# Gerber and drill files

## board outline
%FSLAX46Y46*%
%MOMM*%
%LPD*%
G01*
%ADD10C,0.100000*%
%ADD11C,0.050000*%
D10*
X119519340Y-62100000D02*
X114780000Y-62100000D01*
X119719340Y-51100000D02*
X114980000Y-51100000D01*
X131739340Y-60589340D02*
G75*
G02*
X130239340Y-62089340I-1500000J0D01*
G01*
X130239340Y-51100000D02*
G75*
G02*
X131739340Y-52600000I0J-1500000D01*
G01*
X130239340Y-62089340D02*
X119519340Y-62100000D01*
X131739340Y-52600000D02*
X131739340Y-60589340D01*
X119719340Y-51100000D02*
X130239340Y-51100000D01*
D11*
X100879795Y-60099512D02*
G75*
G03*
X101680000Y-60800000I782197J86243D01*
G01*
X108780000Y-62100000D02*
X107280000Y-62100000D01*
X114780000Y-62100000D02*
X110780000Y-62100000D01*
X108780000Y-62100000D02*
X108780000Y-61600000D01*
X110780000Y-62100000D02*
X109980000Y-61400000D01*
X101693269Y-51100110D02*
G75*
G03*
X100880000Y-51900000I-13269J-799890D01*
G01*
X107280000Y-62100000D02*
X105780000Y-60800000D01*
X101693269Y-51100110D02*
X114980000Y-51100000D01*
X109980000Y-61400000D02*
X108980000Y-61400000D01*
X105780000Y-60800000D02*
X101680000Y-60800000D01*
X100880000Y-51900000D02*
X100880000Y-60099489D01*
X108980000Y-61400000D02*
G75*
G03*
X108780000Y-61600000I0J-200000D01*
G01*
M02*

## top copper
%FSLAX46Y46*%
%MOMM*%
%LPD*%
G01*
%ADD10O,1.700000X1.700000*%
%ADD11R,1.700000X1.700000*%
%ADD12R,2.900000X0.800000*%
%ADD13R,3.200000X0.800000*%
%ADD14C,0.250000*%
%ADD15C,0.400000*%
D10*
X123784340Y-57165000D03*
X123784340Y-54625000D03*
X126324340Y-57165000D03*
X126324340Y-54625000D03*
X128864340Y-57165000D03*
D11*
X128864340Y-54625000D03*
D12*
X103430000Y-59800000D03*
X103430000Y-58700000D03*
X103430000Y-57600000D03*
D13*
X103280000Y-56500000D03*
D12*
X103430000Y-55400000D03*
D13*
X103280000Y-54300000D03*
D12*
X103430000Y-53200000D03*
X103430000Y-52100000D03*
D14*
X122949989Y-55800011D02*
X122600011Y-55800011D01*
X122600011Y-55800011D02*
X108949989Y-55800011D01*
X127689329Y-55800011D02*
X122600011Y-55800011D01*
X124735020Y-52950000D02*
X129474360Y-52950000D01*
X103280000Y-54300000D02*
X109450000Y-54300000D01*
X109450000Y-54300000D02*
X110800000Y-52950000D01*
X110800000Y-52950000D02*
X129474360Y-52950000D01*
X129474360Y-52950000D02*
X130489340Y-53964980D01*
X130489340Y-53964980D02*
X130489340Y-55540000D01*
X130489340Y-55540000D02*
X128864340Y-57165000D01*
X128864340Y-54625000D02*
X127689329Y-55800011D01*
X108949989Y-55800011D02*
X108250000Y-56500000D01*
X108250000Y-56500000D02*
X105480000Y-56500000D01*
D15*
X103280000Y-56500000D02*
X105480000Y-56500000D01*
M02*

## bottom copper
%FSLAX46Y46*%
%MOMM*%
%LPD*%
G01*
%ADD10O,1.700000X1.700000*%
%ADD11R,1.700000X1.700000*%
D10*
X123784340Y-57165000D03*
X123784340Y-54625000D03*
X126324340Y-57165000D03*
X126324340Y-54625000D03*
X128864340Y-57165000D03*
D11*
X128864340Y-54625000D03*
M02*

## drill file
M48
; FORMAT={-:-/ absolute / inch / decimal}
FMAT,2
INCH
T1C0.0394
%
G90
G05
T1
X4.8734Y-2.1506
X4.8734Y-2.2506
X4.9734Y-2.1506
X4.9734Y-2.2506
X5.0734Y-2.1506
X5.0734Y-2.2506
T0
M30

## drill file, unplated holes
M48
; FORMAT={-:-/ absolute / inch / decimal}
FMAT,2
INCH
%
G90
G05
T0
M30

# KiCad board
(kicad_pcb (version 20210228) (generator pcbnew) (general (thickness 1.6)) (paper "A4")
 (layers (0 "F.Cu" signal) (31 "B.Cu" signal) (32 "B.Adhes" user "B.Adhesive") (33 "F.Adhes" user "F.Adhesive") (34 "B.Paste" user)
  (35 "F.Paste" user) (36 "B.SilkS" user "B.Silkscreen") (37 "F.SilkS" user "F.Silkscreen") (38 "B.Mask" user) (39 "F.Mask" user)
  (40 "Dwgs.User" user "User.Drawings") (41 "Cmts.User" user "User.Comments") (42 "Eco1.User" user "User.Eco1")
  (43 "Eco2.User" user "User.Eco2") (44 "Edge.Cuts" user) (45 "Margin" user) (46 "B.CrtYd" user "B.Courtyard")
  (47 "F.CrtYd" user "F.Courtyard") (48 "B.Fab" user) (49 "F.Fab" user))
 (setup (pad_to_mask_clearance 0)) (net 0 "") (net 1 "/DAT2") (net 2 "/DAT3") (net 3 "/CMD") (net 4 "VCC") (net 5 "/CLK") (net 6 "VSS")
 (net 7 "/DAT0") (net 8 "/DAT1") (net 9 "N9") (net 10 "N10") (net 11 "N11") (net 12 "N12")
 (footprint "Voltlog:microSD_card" (layer "F.Cu") (at 109.63 55.95 90)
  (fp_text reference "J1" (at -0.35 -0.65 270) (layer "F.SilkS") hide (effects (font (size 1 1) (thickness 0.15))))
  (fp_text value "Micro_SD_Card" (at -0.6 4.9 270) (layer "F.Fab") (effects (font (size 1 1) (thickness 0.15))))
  (pad "1" smd rect (at -3.85 -6.2 90) (locked) (size 0.8 2.9) (layers "F.Cu" "F.Mask") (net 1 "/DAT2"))
  (pad "2" smd rect (at -2.75 -6.2 90) (locked) (size 0.8 2.9) (layers "F.Cu" "F.Mask") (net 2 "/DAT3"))
  (pad "3" smd rect (at -1.65 -6.2 90) (locked) (size 0.8 2.9) (layers "F.Cu" "F.Mask") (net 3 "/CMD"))
  (pad "4" smd rect (at -0.55 -6.35 90) (locked) (size 0.8 3.2) (layers "F.Cu" "F.Mask") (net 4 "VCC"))
  (pad "5" smd rect (at 0.55 -6.2 90) (locked) (size 0.8 2.9) (layers "F.Cu" "F.Mask") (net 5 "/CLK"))
  (pad "6" smd rect (at 1.65 -6.35 90) (locked) (size 0.8 3.2) (layers "F.Cu" "F.Mask") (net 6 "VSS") (zone_connect 2))
  (pad "7" smd rect (at 2.75 -6.2 90) (locked) (size 0.8 2.9) (layers "F.Cu" "F.Mask") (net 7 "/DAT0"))
  (pad "8" smd rect (at 3.85 -6.2 90) (locked) (size 0.8 2.9) (layers "F.Cu" "F.Mask") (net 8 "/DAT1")))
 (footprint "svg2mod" (layer "F.Cu") (at 115.55 56.15)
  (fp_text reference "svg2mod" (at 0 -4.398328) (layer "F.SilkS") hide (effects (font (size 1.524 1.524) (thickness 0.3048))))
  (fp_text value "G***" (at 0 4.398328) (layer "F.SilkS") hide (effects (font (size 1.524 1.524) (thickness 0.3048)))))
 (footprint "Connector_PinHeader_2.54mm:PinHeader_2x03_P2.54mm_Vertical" (layer "F.Cu") (at 128.86434 54.625 -90)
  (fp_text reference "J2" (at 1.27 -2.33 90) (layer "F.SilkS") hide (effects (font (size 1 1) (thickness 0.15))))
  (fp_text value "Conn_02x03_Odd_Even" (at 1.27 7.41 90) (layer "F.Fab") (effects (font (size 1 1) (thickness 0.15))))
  (pad "1" thru_hole rect (at 0 0 270) (locked) (size 1.7 1.7) (drill 1) (layers *.Cu *.Mask) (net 4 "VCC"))
  (pad "2" thru_hole oval (at 2.54 0 270) (locked) (size 1.7 1.7) (drill 1) (layers *.Cu *.Mask) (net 6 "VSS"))
  (pad "3" thru_hole oval (at 0 2.54 270) (locked) (size 1.7 1.7) (drill 1) (layers *.Cu *.Mask) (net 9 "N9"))
  (pad "4" thru_hole oval (at 2.54 2.54 270) (locked) (size 1.7 1.7) (drill 1) (layers *.Cu *.Mask) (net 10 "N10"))
  (pad "5" thru_hole oval (at 0 5.08 270) (locked) (size 1.7 1.7) (drill 1) (layers *.Cu *.Mask) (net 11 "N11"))
  (pad "6" thru_hole oval (at 2.54 5.08 270) (locked) (size 1.7 1.7) (drill 1) (layers *.Cu *.Mask) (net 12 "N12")))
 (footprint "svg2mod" (layer "F.Cu") (at 121.35 60.4)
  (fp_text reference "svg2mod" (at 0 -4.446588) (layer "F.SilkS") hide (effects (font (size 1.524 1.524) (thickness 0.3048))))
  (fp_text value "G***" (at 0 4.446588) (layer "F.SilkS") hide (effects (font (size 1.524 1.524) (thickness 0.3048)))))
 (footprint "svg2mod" (layer "F.Cu") (at 115.55 53.35)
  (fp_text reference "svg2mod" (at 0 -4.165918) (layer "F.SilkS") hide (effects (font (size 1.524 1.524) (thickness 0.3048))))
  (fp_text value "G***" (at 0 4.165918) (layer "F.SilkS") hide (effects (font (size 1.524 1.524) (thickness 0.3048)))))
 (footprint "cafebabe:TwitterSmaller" (layer "B.Cu") (at 120.4 60 180)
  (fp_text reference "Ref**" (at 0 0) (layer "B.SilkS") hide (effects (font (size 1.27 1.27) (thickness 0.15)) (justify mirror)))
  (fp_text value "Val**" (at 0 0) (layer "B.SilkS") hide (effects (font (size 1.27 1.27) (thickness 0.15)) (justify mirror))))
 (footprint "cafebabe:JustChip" (layer "B.Cu") (at 113 55.9 180)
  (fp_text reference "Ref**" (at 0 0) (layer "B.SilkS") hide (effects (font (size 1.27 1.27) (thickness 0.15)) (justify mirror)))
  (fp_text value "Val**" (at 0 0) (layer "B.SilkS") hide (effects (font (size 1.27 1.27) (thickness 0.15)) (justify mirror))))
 (gr_arc (start 101.661992 60.013269) (end 101.68 60.8) (angle 85.01938241) (layer "Edge.Cuts") (width 0.05))
 (gr_line (start 108.78 62.1) (end 107.28 62.1) (layer "Edge.Cuts") (width 0.05))
 (gr_line (start 119.71934 51.1) (end 114.98 51.1) (layer "Edge.Cuts") (width 0.1))
 (gr_line (start 119.71934 51.1) (end 130.23934 51.1) (layer "Edge.Cuts") (width 0.1))
 (gr_line (start 119.51934 62.1) (end 114.78 62.1) (layer "Edge.Cuts") (width 0.1))
 (gr_line (start 114.78 62.1) (end 110.78 62.1) (layer "Edge.Cuts") (width 0.05))
 (gr_arc (start 130.23934 60.58934) (end 130.23934 62.08934) (angle -90) (layer "Edge.Cuts") (width 0.1))
 (gr_line (start 108.78 62.1) (end 108.78 61.6) (layer "Edge.Cuts") (width 0.05))
 (gr_line (start 110.78 62.1) (end 109.98 61.4) (layer "Edge.Cuts") (width 0.05))
 (gr_arc (start 101.68 51.9) (end 100.88 51.9) (angle 90.95033288) (layer "Edge.Cuts") (width 0.05))
 (gr_line (start 107.28 62.1) (end 105.78 60.8) (layer "Edge.Cuts") (width 0.05))
 (gr_line (start 101.693269 51.10011) (end 114.98 51.1) (layer "Edge.Cuts") (width 0.05))
 (gr_line (start 109.98 61.4) (end 108.98 61.4) (layer "Edge.Cuts") (width 0.05))
 (gr_line (start 105.78 60.8) (end 101.68 60.8) (layer "Edge.Cuts") (width 0.05))
 (gr_line (start 131.73934 52.6) (end 131.73934 60.58934) (layer "Edge.Cuts") (width 0.1))
 (gr_arc (start 130.23934 52.6) (end 131.73934 52.6) (angle -90) (layer "Edge.Cuts") (width 0.1))
 (gr_line (start 100.88 51.9) (end 100.88 60.099489) (layer "Edge.Cuts") (width 0.05))
 (gr_arc (start 108.98 61.6) (end 108.78 61.6) (angle 90) (layer "Edge.Cuts") (width 0.05))
 (gr_line (start 130.23934 62.08934) (end 119.51934 62.1) (layer "Edge.Cuts") (width 0.1))
 (segment (start 122.949989 55.800011) (end 122.600011 55.800011) (width 0.25) (layer "F.Cu") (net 4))
 (segment (start 128.86434 54.625) (end 127.689329 55.800011) (width 0.25) (layer "F.Cu") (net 4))
 (segment (start 127.689329 55.800011) (end 122.600011 55.800011) (width 0.25) (layer "F.Cu") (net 4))
 (segment (start 122.600011 55.800011) (end 108.949989 55.800011) (width 0.25) (layer "F.Cu") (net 4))
 (segment (start 108.25 56.5) (end 105.48 56.5) (width 0.25) (layer "F.Cu") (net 4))
 (segment (start 108.949989 55.800011) (end 108.25 56.5) (width 0.25) (layer "F.Cu") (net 4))
 (segment (start 103.28 56.5) (end 105.48 56.5) (width 0.4) (layer "F.Cu") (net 4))
 (segment (start 109.45 54.3) (end 110.8 52.95) (width 0.25) (layer "F.Cu") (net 6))
 (segment (start 103.28 54.3) (end 109.45 54.3) (width 0.25) (layer "F.Cu") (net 6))
 (segment (start 124.73502 52.95) (end 129.47436 52.95) (width 0.25) (layer "F.Cu") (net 6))
 (segment (start 110.8 52.95) (end 129.47436 52.95) (width 0.25) (layer "F.Cu") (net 6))
 (segment (start 129.47436 52.95) (end 130.48934 53.96498) (width 0.25) (layer "F.Cu") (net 6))
 (segment (start 130.48934 53.96498) (end 130.48934 55.54) (width 0.25) (layer "F.Cu") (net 6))
 (segment (start 130.48934 55.54) (end 128.86434 57.165) (width 0.25) (layer "F.Cu") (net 6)))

